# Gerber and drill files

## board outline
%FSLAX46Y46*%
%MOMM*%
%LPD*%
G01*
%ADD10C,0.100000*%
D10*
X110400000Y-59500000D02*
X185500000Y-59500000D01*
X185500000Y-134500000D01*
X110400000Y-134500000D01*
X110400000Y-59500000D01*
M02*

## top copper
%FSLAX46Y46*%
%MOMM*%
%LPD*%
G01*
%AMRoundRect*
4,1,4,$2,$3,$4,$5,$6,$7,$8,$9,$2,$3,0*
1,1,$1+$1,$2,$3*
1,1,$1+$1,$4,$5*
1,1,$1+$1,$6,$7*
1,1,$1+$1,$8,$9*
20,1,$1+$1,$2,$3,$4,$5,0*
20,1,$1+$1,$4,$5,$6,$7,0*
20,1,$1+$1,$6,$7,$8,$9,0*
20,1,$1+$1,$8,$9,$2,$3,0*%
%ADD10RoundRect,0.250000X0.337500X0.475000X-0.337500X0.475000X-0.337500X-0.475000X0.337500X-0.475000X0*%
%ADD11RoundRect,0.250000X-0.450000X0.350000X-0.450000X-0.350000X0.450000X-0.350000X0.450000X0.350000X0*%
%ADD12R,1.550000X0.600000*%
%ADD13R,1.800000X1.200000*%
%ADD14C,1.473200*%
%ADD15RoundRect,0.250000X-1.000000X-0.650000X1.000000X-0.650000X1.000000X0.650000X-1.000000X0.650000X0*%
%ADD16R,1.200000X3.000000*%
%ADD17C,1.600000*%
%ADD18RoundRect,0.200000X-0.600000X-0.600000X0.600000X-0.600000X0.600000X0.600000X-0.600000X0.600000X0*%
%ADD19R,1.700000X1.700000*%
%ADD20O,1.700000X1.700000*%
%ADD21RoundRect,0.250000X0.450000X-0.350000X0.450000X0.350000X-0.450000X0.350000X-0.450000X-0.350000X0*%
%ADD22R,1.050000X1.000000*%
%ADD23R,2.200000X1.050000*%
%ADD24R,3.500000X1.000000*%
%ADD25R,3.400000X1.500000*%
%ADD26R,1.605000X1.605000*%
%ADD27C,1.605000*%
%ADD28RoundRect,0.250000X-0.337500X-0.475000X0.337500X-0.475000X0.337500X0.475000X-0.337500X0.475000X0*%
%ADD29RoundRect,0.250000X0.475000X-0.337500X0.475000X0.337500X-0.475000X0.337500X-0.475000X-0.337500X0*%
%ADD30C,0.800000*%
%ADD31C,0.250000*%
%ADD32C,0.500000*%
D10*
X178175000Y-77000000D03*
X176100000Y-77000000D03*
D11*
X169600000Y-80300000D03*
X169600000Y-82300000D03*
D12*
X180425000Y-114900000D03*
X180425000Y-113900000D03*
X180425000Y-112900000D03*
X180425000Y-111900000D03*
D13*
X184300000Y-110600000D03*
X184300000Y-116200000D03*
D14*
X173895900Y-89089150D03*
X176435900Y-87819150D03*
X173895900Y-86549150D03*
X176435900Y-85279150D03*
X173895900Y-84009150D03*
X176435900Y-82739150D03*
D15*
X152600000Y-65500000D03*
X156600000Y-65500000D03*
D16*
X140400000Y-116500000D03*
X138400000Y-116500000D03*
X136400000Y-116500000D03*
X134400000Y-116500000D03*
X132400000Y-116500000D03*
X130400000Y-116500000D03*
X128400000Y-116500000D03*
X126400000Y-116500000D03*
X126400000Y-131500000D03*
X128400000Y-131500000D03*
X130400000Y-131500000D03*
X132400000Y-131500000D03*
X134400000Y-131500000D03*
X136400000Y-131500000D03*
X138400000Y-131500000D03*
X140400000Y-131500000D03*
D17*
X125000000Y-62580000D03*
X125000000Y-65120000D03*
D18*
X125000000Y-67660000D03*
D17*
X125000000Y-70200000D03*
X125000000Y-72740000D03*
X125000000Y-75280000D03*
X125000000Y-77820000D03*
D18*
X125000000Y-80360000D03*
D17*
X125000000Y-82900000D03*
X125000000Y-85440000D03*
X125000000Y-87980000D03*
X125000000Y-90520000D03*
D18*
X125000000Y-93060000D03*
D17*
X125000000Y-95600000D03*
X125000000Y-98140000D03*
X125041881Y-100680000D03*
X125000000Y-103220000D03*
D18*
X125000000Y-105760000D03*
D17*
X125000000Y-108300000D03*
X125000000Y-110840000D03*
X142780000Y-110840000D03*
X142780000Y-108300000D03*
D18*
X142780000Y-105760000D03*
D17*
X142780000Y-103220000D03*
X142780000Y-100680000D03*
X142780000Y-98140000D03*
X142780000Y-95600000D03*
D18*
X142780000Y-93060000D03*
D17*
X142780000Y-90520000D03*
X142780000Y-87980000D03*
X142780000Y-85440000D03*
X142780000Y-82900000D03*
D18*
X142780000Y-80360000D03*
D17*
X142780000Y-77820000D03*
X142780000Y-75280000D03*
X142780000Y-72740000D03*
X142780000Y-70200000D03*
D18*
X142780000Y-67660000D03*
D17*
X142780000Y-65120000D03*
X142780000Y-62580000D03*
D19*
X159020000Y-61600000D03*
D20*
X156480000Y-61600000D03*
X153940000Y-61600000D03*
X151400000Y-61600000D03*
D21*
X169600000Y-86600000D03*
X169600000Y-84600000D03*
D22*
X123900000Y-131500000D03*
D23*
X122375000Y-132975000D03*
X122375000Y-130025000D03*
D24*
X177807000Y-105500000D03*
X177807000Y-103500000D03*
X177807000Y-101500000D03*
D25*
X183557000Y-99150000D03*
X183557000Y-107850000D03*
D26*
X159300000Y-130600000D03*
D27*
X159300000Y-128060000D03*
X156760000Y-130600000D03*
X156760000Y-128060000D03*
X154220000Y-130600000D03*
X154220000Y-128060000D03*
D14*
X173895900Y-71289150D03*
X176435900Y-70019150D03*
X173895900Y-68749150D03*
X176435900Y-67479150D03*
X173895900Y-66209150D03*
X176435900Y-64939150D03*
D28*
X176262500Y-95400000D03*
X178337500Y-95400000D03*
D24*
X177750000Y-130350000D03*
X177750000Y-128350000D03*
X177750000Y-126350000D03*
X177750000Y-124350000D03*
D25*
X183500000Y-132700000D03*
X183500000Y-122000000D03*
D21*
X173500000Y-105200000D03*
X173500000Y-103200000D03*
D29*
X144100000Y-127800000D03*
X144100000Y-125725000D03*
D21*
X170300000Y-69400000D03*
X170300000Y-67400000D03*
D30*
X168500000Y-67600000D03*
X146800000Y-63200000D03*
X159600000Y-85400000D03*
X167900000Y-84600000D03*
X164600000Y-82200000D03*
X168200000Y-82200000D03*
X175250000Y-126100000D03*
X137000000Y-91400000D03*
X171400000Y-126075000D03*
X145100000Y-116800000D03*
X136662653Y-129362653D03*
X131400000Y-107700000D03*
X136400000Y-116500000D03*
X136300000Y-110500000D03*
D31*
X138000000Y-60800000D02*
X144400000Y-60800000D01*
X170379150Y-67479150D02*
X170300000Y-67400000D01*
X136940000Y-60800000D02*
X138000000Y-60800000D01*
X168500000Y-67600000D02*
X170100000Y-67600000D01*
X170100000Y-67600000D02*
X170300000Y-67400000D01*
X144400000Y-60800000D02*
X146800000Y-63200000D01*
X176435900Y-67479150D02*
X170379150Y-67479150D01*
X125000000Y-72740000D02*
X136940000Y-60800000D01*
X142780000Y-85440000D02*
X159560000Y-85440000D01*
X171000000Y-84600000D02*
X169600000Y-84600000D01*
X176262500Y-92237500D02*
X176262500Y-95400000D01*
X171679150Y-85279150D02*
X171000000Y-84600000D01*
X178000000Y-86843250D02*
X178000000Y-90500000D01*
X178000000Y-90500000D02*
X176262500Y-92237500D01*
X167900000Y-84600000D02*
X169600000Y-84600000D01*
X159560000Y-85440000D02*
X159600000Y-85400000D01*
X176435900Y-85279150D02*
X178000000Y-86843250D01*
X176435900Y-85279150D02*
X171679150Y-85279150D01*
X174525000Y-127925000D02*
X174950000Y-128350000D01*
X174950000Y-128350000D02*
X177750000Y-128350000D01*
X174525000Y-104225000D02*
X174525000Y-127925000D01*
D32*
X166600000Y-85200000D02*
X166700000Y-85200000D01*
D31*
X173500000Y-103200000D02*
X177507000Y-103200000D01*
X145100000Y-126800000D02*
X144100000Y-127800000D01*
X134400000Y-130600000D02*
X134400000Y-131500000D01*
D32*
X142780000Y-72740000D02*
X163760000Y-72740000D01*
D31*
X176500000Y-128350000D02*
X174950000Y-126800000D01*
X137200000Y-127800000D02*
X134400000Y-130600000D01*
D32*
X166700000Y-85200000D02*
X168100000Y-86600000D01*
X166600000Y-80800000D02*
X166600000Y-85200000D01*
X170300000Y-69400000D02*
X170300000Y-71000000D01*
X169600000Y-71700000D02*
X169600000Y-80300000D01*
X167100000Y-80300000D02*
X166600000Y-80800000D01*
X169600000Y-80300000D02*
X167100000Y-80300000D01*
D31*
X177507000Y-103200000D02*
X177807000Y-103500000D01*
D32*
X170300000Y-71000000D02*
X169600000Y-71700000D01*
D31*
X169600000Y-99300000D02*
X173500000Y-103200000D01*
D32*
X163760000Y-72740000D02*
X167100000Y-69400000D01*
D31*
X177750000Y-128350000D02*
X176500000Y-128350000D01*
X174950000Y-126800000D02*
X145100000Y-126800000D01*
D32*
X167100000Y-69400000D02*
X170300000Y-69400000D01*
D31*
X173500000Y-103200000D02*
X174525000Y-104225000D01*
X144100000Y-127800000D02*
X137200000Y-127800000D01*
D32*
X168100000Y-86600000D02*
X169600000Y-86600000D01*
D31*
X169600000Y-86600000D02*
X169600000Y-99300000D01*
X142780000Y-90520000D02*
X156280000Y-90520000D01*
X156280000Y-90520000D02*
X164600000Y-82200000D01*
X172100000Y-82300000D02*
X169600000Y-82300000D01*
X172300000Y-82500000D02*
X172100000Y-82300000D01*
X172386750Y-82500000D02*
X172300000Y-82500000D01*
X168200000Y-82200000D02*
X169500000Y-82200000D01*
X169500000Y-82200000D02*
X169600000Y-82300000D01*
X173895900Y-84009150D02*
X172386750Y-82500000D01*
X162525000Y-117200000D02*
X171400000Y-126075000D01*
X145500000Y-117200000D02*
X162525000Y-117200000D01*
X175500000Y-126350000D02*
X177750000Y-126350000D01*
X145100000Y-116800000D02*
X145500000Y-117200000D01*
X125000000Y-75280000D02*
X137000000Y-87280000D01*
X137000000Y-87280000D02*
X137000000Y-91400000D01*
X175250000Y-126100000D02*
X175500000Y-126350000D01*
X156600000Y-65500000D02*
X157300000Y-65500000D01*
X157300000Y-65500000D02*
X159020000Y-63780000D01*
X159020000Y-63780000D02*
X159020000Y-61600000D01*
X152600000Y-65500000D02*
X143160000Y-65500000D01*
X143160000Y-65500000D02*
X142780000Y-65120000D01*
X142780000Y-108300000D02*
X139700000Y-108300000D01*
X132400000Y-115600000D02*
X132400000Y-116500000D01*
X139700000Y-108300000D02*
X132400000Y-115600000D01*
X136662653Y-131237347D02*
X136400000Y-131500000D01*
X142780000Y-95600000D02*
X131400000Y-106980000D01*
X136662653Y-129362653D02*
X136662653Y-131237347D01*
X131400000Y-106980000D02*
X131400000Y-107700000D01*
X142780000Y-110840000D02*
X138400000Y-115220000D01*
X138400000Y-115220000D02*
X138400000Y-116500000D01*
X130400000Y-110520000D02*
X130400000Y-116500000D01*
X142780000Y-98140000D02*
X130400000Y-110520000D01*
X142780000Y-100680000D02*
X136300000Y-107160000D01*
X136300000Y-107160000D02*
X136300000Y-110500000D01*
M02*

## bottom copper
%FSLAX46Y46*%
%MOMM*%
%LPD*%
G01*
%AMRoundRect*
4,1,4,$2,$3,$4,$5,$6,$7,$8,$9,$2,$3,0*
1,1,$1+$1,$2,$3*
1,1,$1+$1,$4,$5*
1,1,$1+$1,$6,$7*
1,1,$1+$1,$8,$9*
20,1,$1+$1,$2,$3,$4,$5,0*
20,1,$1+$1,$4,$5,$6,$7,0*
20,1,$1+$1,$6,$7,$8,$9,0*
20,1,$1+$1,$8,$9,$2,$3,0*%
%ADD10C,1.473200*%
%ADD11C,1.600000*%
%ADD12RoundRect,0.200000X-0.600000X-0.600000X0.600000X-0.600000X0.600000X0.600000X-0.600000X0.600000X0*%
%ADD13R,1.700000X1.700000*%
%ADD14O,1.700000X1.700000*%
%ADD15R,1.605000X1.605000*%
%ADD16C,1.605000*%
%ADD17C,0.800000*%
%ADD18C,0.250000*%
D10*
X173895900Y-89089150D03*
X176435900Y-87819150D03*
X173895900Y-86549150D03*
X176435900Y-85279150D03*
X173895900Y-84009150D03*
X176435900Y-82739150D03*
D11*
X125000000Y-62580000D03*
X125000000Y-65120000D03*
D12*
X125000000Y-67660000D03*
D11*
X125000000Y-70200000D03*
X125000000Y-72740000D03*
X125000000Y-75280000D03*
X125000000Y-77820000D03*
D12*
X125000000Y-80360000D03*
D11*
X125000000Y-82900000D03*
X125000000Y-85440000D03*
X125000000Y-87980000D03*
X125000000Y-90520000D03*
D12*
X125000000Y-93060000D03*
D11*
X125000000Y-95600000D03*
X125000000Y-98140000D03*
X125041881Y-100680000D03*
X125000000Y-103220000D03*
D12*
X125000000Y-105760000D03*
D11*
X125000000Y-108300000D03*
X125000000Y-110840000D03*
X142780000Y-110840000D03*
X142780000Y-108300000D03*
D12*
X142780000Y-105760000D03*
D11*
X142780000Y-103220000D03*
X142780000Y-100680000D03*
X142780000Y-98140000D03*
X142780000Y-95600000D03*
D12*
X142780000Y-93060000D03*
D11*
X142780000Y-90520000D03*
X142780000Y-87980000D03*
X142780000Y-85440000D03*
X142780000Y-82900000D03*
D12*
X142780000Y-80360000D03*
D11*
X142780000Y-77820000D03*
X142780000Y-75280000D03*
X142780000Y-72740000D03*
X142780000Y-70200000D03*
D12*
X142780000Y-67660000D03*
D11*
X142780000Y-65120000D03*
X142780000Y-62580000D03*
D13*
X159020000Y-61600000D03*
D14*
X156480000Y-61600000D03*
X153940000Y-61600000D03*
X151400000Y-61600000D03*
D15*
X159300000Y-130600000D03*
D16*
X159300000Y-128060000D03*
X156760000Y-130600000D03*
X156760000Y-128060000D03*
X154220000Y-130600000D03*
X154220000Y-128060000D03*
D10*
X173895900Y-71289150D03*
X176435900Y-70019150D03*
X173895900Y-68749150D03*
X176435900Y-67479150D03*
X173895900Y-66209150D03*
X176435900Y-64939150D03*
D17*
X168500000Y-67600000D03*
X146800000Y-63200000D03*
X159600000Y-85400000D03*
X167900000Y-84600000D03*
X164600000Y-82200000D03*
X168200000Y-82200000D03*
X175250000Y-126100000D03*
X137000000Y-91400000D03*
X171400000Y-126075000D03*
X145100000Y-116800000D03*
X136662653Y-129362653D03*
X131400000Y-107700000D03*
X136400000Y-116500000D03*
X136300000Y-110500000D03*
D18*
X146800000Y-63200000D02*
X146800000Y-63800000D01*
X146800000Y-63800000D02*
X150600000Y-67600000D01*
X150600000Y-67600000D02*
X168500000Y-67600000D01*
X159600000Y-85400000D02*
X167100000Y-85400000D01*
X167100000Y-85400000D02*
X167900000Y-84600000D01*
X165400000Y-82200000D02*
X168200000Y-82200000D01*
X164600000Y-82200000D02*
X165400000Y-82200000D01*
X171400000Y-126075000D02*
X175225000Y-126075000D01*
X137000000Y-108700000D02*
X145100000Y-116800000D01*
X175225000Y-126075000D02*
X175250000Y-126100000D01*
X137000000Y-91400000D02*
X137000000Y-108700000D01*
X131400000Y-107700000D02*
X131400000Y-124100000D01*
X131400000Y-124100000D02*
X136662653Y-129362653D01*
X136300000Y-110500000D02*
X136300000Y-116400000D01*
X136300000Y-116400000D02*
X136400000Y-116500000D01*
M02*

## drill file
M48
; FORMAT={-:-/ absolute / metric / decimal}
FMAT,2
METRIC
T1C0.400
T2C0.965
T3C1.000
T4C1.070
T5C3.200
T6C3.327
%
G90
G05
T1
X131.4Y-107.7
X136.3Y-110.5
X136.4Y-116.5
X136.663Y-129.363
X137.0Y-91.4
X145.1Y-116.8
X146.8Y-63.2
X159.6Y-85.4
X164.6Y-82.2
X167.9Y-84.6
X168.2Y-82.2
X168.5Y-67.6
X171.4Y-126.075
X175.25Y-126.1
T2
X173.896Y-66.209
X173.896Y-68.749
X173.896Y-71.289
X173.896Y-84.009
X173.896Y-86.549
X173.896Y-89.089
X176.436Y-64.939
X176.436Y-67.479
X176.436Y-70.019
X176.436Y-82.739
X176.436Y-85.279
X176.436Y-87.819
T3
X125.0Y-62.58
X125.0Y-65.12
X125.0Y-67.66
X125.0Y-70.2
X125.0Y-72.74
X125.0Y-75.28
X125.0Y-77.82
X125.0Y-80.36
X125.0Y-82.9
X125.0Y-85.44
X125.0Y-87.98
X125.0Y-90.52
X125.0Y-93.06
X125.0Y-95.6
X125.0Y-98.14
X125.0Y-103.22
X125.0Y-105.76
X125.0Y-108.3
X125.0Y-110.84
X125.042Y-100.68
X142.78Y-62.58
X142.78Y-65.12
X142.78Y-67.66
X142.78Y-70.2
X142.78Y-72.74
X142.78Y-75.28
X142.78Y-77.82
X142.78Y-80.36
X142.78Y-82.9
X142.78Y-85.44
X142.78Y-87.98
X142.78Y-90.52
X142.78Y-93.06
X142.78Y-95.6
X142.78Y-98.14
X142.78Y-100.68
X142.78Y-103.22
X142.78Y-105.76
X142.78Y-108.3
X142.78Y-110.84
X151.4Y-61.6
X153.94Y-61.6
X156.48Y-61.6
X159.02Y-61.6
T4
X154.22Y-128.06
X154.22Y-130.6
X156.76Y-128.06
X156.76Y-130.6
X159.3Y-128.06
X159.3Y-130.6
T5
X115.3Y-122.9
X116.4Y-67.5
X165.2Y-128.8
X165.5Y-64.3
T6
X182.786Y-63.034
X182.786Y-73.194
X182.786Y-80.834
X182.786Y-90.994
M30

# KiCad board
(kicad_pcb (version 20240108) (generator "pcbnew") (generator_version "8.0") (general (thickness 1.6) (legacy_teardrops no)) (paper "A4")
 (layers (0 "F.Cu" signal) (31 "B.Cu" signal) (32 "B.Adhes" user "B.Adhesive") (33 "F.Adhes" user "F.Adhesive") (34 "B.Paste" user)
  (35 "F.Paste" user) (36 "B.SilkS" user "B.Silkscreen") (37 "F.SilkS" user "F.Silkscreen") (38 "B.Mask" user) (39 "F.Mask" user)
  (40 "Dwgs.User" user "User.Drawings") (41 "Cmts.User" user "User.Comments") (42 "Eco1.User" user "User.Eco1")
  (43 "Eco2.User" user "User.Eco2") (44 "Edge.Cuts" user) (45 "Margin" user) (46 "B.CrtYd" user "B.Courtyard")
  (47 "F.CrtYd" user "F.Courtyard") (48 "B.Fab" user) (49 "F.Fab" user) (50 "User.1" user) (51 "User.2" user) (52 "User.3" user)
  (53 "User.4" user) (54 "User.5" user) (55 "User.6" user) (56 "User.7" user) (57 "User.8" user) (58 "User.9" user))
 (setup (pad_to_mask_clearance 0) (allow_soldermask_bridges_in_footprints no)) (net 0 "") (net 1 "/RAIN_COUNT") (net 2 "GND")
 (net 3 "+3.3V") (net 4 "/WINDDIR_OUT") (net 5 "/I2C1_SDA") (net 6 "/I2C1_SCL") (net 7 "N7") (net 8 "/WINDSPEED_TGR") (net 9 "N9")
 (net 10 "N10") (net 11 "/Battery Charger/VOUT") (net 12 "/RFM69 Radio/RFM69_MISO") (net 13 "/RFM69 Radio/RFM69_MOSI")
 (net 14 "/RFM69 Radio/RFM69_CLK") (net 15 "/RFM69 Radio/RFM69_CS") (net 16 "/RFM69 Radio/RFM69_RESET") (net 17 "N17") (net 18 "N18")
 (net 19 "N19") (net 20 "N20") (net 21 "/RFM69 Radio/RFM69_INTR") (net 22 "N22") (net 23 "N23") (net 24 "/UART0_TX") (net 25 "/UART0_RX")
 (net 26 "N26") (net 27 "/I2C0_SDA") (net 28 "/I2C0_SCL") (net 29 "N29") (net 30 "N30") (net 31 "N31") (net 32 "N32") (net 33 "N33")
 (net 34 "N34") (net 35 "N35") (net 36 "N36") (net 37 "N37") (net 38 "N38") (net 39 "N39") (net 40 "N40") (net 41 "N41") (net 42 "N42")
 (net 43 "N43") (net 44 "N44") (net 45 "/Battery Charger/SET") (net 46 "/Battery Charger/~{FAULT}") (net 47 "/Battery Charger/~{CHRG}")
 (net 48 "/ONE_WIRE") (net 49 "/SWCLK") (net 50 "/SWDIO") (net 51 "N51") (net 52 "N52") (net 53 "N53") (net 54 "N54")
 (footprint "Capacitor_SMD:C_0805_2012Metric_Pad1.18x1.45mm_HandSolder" (layer "F.Cu") (at 177.1375 77 180)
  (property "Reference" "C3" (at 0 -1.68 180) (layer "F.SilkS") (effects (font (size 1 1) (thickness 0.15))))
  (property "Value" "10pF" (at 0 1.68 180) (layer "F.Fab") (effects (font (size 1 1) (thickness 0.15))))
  (pad "1" smd roundrect (at -1.0375 0 180) (size 1.175 1.45) (layers "F.Cu" "F.Paste" "F.Mask") (roundrect_rratio 0.212766)
   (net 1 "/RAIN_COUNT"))
  (pad "2" smd roundrect (at 1.0375 0 180) (size 1.175 1.45) (layers "F.Cu" "F.Paste" "F.Mask") (roundrect_rratio 0.212766) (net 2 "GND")))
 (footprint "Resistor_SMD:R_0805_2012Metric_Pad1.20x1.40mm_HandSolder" (layer "F.Cu") (at 169.6 81.3 -90)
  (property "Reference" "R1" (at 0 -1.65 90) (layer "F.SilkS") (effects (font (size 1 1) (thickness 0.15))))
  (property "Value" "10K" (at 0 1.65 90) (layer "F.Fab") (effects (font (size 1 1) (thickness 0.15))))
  (pad "1" smd roundrect (at -1 0 270) (size 1.2 1.4) (layers "F.Cu" "F.Paste" "F.Mask") (roundrect_rratio 0.208333) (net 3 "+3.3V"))
  (pad "2" smd roundrect (at 1 0 270) (size 1.2 1.4) (layers "F.Cu" "F.Paste" "F.Mask") (roundrect_rratio 0.208333) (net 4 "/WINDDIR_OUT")))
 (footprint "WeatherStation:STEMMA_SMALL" (layer "F.Cu") (at 181.2 113.4 90)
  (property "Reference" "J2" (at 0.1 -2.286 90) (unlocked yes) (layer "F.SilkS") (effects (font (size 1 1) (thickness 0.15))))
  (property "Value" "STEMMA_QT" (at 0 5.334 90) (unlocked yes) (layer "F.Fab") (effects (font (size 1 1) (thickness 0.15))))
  (pad "1" smd rect (at -1.5 -0.775 90) (size 0.6 1.55) (layers "F.Cu" "F.Paste" "F.Mask") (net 2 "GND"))
  (pad "2" smd rect (at -0.5 -0.775 90) (size 0.6 1.55) (layers "F.Cu" "F.Paste" "F.Mask") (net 3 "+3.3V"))
  (pad "3" smd rect (at 0.5 -0.775 90) (size 0.6 1.55) (layers "F.Cu" "F.Paste" "F.Mask") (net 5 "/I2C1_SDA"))
  (pad "4" smd rect (at 1.5 -0.775 90) (size 0.6 1.55) (layers "F.Cu" "F.Paste" "F.Mask") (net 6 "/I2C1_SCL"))
  (pad "5" smd rect (at 2.8 3.1 90) (size 1.2 1.8) (layers "F.Cu" "F.Paste" "F.Mask"))
  (pad "6" smd rect (at -2.8 3.1 90) (size 1.2 1.8) (layers "F.Cu" "F.Paste" "F.Mask")))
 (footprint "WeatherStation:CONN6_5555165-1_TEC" (layer "F.Cu") (at 173.8959 89.08915 90)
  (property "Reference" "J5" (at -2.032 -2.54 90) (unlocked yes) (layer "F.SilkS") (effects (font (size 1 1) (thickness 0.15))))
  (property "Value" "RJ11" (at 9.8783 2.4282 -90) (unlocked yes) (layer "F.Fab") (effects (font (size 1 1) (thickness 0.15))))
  (pad "" np_thru_hole circle (at -1.905 8.89 90) (size 3.3274 3.3274) (drill 3.3274) (layers "*.Cu" "*.Mask"))
  (pad "" np_thru_hole circle (at 8.255 8.89 90) (size 3.3274 3.3274) (drill 3.3274) (layers "*.Cu" "*.Mask"))
  (pad "1" thru_hole circle (at 0 0 90) (size 1.4732 1.4732) (drill 0.9652) (layers "*.Cu" "*.Mask") (remove_unused_layers no) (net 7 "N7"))
  (pad "2" thru_hole circle (at 1.27 2.54 90) (size 1.4732 1.4732) (drill 0.9652) (layers "*.Cu" "*.Mask") (remove_unused_layers no)
   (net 2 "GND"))
  (pad "3" thru_hole circle (at 2.54 0 90) (size 1.4732 1.4732) (drill 0.9652) (layers "*.Cu" "*.Mask") (remove_unused_layers no)
   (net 2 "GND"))
  (pad "4" thru_hole circle (at 3.81 2.54 90) (size 1.4732 1.4732) (drill 0.9652) (layers "*.Cu" "*.Mask") (remove_unused_layers no)
   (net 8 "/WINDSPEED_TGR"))
  (pad "5" thru_hole circle (at 5.08 0 90) (size 1.4732 1.4732) (drill 0.9652) (layers "*.Cu" "*.Mask") (remove_unused_layers no)
   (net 4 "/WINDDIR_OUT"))
  (pad "6" thru_hole circle (at 6.35 2.54 90) (size 1.4732 1.4732) (drill 0.9652) (layers "*.Cu" "*.Mask") (remove_unused_layers no)
   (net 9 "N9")))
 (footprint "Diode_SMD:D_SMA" (layer "F.Cu") (at 154.6 65.5)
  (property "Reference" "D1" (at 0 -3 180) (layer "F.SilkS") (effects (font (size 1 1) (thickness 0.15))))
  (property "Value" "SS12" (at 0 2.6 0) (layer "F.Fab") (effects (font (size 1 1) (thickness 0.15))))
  (pad "1" smd roundrect (at -2 0) (size 2.5 1.8) (layers "F.Cu" "F.Paste" "F.Mask") (roundrect_rratio 0.1388888889) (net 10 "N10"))
  (pad "2" smd roundrect (at 2 0) (size 2.5 1.8) (layers "F.Cu" "F.Paste" "F.Mask") (roundrect_rratio 0.1388888889)
   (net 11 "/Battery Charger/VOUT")))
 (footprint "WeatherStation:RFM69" (layer "F.Cu") (at 133.4 124 -90)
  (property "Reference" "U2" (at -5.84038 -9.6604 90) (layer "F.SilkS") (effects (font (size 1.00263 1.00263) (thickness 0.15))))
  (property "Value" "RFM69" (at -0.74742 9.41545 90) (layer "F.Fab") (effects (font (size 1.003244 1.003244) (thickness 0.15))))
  (pad "1" smd rect (at -7.5 -7 270) (size 3 1.2) (layers "F.Cu" "F.Paste" "F.Mask") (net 2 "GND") (solder_mask_margin 0.102))
  (pad "2" smd rect (at -7.5 -5 270) (size 3 1.2) (layers "F.Cu" "F.Paste" "F.Mask") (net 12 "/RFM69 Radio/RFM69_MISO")
   (solder_mask_margin 0.102))
  (pad "3" smd rect (at -7.5 -3 270) (size 3 1.2) (layers "F.Cu" "F.Paste" "F.Mask") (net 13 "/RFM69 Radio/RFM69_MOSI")
   (solder_mask_margin 0.102))
  (pad "4" smd rect (at -7.5 -1 270) (size 3 1.2) (layers "F.Cu" "F.Paste" "F.Mask") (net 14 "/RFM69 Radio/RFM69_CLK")
   (solder_mask_margin 0.102))
  (pad "5" smd rect (at -7.5 1 270) (size 3 1.2) (layers "F.Cu" "F.Paste" "F.Mask") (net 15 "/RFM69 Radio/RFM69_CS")
   (solder_mask_margin 0.102))
  (pad "6" smd rect (at -7.5 3 270) (size 3 1.2) (layers "F.Cu" "F.Paste" "F.Mask") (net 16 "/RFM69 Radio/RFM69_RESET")
   (solder_mask_margin 0.102))
  (pad "7" smd rect (at -7.5 5 270) (size 3 1.2) (layers "F.Cu" "F.Paste" "F.Mask") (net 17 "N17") (solder_mask_margin 0.102))
  (pad "8" smd rect (at -7.5 7 270) (size 3 1.2) (layers "F.Cu" "F.Paste" "F.Mask") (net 2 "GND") (solder_mask_margin 0.102))
  (pad "9" smd rect (at 7.5 7 270) (size 3 1.2) (layers "F.Cu" "F.Paste" "F.Mask") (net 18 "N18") (solder_mask_margin 0.102))
  (pad "10" smd rect (at 7.5 5 270) (size 3 1.2) (layers "F.Cu" "F.Paste" "F.Mask") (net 2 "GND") (solder_mask_margin 0.102))
  (pad "11" smd rect (at 7.5 3 270) (size 3 1.2) (layers "F.Cu" "F.Paste" "F.Mask") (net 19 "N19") (solder_mask_margin 0.102))
  (pad "12" smd rect (at 7.5 1 270) (size 3 1.2) (layers "F.Cu" "F.Paste" "F.Mask") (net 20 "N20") (solder_mask_margin 0.102))
  (pad "13" smd rect (at 7.5 -1 270) (size 3 1.2) (layers "F.Cu" "F.Paste" "F.Mask") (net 3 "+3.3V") (solder_mask_margin 0.102))
  (pad "14" smd rect (at 7.5 -3 270) (size 3 1.2) (layers "F.Cu" "F.Paste" "F.Mask") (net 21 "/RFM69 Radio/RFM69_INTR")
   (solder_mask_margin 0.102))
  (pad "15" smd rect (at 7.5 -5 270) (size 3 1.2) (layers "F.Cu" "F.Paste" "F.Mask") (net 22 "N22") (solder_mask_margin 0.102))
  (pad "16" smd rect (at 7.5 -7 270) (size 3 1.2) (layers "F.Cu" "F.Paste" "F.Mask") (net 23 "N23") (solder_mask_margin 0.102)))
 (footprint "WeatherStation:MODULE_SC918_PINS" (layer "F.Cu") (at 133.89 86.71)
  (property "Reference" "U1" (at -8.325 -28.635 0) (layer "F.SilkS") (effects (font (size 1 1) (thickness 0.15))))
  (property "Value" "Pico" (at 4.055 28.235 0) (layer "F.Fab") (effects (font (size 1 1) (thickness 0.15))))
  (pad "1" thru_hole circle (at -8.89 -24.13) (size 1.6 1.6) (drill 1) (layers "*.Cu" "*.Mask") (remove_unused_layers no)
   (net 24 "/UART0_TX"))
  (pad "2" thru_hole circle (at -8.89 -21.59) (size 1.6 1.6) (drill 1) (layers "*.Cu" "*.Mask") (remove_unused_layers no)
   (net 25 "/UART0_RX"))
  (pad "3" thru_hole roundrect (at -8.89 -19.05) (size 1.6 1.6) (drill 1) (layers "*.Cu" "*.Mask") (remove_unused_layers no)
   (roundrect_rratio 0.125) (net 2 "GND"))
  (pad "4" thru_hole circle (at -8.89 -16.51) (size 1.6 1.6) (drill 1) (layers "*.Cu" "*.Mask") (remove_unused_layers no) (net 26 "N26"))
  (pad "5" thru_hole circle (at -8.89 -13.97) (size 1.6 1.6) (drill 1) (layers "*.Cu" "*.Mask") (remove_unused_layers no)
   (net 1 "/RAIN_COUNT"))
  (pad "6" thru_hole circle (at -8.89 -11.43) (size 1.6 1.6) (drill 1) (layers "*.Cu" "*.Mask") (remove_unused_layers no)
   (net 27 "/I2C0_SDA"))
  (pad "7" thru_hole circle (at -8.89 -8.89) (size 1.6 1.6) (drill 1) (layers "*.Cu" "*.Mask") (remove_unused_layers no)
   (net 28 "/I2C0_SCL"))
  (pad "8" thru_hole roundrect (at -8.89 -6.35) (size 1.6 1.6) (drill 1) (layers "*.Cu" "*.Mask") (remove_unused_layers no)
   (roundrect_rratio 0.125) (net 2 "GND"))
  (pad "9" thru_hole circle (at -8.89 -3.81) (size 1.6 1.6) (drill 1) (layers "*.Cu" "*.Mask") (remove_unused_layers no) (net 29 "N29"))
  (pad "10" thru_hole circle (at -8.89 -1.27) (size 1.6 1.6) (drill 1) (layers "*.Cu" "*.Mask") (remove_unused_layers no) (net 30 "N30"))
  (pad "11" thru_hole circle (at -8.89 1.27) (size 1.6 1.6) (drill 1) (layers "*.Cu" "*.Mask") (remove_unused_layers no) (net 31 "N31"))
  (pad "12" thru_hole circle (at -8.89 3.81) (size 1.6 1.6) (drill 1) (layers "*.Cu" "*.Mask") (remove_unused_layers no) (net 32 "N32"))
  (pad "13" thru_hole roundrect (at -8.89 6.35) (size 1.6 1.6) (drill 1) (layers "*.Cu" "*.Mask") (remove_unused_layers no)
   (roundrect_rratio 0.125) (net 2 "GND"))
  (pad "14" thru_hole circle (at -8.89 8.89) (size 1.6 1.6) (drill 1) (layers "*.Cu" "*.Mask") (remove_unused_layers no) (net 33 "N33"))
  (pad "15" thru_hole circle (at -8.89 11.43) (size 1.6 1.6) (drill 1) (layers "*.Cu" "*.Mask") (remove_unused_layers no) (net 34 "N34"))
  (pad "16" thru_hole circle (at -8.848119 13.97) (size 1.6 1.6) (drill 1) (layers "*.Cu" "*.Mask") (remove_unused_layers no) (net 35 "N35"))
  (pad "17" thru_hole circle (at -8.89 16.51) (size 1.6 1.6) (drill 1) (layers "*.Cu" "*.Mask") (remove_unused_layers no) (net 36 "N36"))
  (pad "18" thru_hole roundrect (at -8.89 19.05) (size 1.6 1.6) (drill 1) (layers "*.Cu" "*.Mask") (remove_unused_layers no)
   (roundrect_rratio 0.125) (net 2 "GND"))
  (pad "19" thru_hole circle (at -8.89 21.59) (size 1.6 1.6) (drill 1) (layers "*.Cu" "*.Mask") (remove_unused_layers no) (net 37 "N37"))
  (pad "20" thru_hole circle (at -8.89 24.13) (size 1.6 1.6) (drill 1) (layers "*.Cu" "*.Mask") (remove_unused_layers no) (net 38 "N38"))
  (pad "21" thru_hole circle (at 8.89 24.13) (size 1.6 1.6) (drill 1) (layers "*.Cu" "*.Mask") (remove_unused_layers no)
   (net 12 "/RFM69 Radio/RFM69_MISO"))
  (pad "22" thru_hole circle (at 8.89 21.59) (size 1.6 1.6) (drill 1) (layers "*.Cu" "*.Mask") (remove_unused_layers no)
   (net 15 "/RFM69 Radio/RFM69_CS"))
  (pad "23" thru_hole roundrect (at 8.89 19.05) (size 1.6 1.6) (drill 1) (layers "*.Cu" "*.Mask") (remove_unused_layers no)
   (roundrect_rratio 0.125) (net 2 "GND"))
  (pad "24" thru_hole circle (at 8.89 16.51) (size 1.6 1.6) (drill 1) (layers "*.Cu" "*.Mask") (remove_unused_layers no)
   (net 14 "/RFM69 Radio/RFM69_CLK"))
  (pad "25" thru_hole circle (at 8.89 13.97) (size 1.6 1.6) (drill 1) (layers "*.Cu" "*.Mask") (remove_unused_layers no)
   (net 13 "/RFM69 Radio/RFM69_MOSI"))
  (pad "26" thru_hole circle (at 8.89 11.43) (size 1.6 1.6) (drill 1) (layers "*.Cu" "*.Mask") (remove_unused_layers no)
   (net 16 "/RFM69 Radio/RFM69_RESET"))
  (pad "27" thru_hole circle (at 8.89 8.89) (size 1.6 1.6) (drill 1) (layers "*.Cu" "*.Mask") (remove_unused_layers no)
   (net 21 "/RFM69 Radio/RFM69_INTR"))
  (pad "28" thru_hole roundrect (at 8.89 6.35) (size 1.6 1.6) (drill 1) (layers "*.Cu" "*.Mask") (remove_unused_layers no)
   (roundrect_rratio 0.125) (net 2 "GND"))
  (pad "29" thru_hole circle (at 8.89 3.81) (size 1.6 1.6) (drill 1) (layers "*.Cu" "*.Mask") (remove_unused_layers no)
   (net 4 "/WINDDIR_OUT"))
  (pad "30" thru_hole circle (at 8.89 1.27) (size 1.6 1.6) (drill 1) (layers "*.Cu" "*.Mask") (remove_unused_layers no) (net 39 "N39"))
  (pad "31" thru_hole circle (at 8.89 -1.27) (size 1.6 1.6) (drill 1) (layers "*.Cu" "*.Mask") (remove_unused_layers no)
   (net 8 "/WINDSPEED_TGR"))
  (pad "32" thru_hole circle (at 8.89 -3.81) (size 1.6 1.6) (drill 1) (layers "*.Cu" "*.Mask") (remove_unused_layers no) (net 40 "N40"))
  (pad "33" thru_hole roundrect (at 8.89 -6.35) (size 1.6 1.6) (drill 1) (layers "*.Cu" "*.Mask") (remove_unused_layers no)
   (roundrect_rratio 0.125) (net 2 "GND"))
  (pad "34" thru_hole circle (at 8.89 -8.89) (size 1.6 1.6) (drill 1) (layers "*.Cu" "*.Mask") (remove_unused_layers no) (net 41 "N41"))
  (pad "35" thru_hole circle (at 8.89 -11.43) (size 1.6 1.6) (drill 1) (layers "*.Cu" "*.Mask") (remove_unused_layers no) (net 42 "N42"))
  (pad "36" thru_hole circle (at 8.89 -13.97) (size 1.6 1.6) (drill 1) (layers "*.Cu" "*.Mask") (remove_unused_layers no) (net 3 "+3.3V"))
  (pad "37" thru_hole circle (at 8.89 -16.51) (size 1.6 1.6) (drill 1) (layers "*.Cu" "*.Mask") (remove_unused_layers no) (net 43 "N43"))
  (pad "38" thru_hole roundrect (at 8.89 -19.05) (size 1.6 1.6) (drill 1) (layers "*.Cu" "*.Mask") (remove_unused_layers no)
   (roundrect_rratio 0.125) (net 2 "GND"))
  (pad "39" thru_hole circle (at 8.89 -21.59) (size 1.6 1.6) (drill 1) (layers "*.Cu" "*.Mask") (remove_unused_layers no) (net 10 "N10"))
  (pad "40" thru_hole circle (at 8.89 -24.13) (size 1.6 1.6) (drill 1) (layers "*.Cu" "*.Mask") (remove_unused_layers no) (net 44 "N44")))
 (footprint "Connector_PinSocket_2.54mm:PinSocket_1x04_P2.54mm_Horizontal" (layer "F.Cu") (at 159.02 61.6 -90)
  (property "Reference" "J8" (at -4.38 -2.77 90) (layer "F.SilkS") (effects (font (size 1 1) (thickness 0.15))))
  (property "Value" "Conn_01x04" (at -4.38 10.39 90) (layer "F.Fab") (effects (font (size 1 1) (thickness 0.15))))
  (pad "1" thru_hole rect (at 0 0 270) (size 1.7 1.7) (drill 1) (layers "*.Cu" "*.Mask") (remove_unused_layers no)
   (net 11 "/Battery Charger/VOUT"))
  (pad "2" thru_hole oval (at 0 2.54 270) (size 1.7 1.7) (drill 1) (layers "*.Cu" "*.Mask") (remove_unused_layers no)
   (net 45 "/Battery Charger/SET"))
  (pad "3" thru_hole oval (at 0 5.08 270) (size 1.7 1.7) (drill 1) (layers "*.Cu" "*.Mask") (remove_unused_layers no)
   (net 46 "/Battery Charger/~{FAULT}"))
  (pad "4" thru_hole oval (at 0 7.62 270) (size 1.7 1.7) (drill 1) (layers "*.Cu" "*.Mask") (remove_unused_layers no)
   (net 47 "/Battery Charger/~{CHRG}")))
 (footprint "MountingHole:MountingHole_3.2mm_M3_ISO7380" (layer "F.Cu") (at 165.2 128.8)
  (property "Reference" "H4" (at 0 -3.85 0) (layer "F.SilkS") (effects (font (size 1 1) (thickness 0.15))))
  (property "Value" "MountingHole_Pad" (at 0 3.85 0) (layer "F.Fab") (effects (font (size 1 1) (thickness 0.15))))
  (pad "" np_thru_hole circle (at 0 0) (size 3.2 3.2) (drill 3.2) (layers "*.Cu" "*.Mask")))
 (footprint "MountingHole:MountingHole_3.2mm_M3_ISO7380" (layer "F.Cu") (at 115.3 122.9)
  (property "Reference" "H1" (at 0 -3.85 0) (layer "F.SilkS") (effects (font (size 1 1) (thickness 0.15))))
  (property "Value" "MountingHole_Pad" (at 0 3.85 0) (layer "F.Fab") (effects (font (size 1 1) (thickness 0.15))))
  (pad "" np_thru_hole circle (at 0 0) (size 3.2 3.2) (drill 3.2) (layers "*.Cu" "*.Mask")))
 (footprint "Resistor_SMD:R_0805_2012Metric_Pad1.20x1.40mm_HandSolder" (layer "F.Cu") (at 169.6 85.6 90)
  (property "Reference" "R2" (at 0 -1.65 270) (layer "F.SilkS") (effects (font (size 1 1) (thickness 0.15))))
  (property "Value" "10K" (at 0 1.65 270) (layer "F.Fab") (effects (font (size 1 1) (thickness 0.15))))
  (pad "1" smd roundrect (at -1 0 90) (size 1.2 1.4) (layers "F.Cu" "F.Paste" "F.Mask") (roundrect_rratio 0.208333) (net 3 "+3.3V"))
  (pad "2" smd roundrect (at 1 0 90) (size 1.2 1.4) (layers "F.Cu" "F.Paste" "F.Mask") (roundrect_rratio 0.208333) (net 8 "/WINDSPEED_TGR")))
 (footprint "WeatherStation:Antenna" (layer "F.Cu") (at 122.375 131.5 90)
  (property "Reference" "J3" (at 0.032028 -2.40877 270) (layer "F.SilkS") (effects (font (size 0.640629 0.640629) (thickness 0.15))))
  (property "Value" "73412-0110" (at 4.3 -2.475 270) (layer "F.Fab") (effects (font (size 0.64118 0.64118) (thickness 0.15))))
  (pad "1" smd rect (at 0 1.525 90) (size 1 1.05) (layers "F.Cu" "F.Paste" "F.Mask") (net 18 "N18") (solder_mask_margin 0.102))
  (pad "2" smd rect (at -1.475 0 90) (size 1.05 2.2) (layers "F.Cu" "F.Paste" "F.Mask") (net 2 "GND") (solder_mask_margin 0.102))
  (pad "3" smd rect (at 1.475 0 90) (size 1.05 2.2) (layers "F.Cu" "F.Paste" "F.Mask") (solder_mask_margin 0.102)))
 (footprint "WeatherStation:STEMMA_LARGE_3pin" (layer "F.Cu") (at 179.557 103.5 90)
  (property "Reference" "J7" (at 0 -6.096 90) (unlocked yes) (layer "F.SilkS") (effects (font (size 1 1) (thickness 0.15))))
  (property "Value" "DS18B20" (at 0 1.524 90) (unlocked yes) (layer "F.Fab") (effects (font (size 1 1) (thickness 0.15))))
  (pad "1" smd rect (at -2 -1.75 90) (size 1 3.5) (layers "F.Cu" "F.Paste" "F.Mask") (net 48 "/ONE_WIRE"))
  (pad "2" smd rect (at 0 -1.75 90) (size 1 3.5) (layers "F.Cu" "F.Paste" "F.Mask") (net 3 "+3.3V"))
  (pad "3" smd rect (at 2 -1.75 90) (size 1 3.5) (layers "F.Cu" "F.Paste" "F.Mask") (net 2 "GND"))
  (pad "4" smd rect (at 4.35 4 90) (size 1.5 3.4) (layers "F.Cu" "F.Paste" "F.Mask"))
  (pad "5" smd rect (at -4.35 4 90) (size 1.5 3.4) (layers "F.Cu" "F.Paste" "F.Mask")))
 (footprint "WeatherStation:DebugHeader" (layer "F.Cu") (at 156.76 129.33)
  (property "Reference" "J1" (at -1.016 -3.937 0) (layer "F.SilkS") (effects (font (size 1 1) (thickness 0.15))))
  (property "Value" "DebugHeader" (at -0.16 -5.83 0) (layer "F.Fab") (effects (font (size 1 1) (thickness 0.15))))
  (pad "1" thru_hole rect (at 2.54 1.27) (size 1.605 1.605) (drill 1.07) (layers "*.Cu" "*.Mask") (remove_unused_layers no)
   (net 24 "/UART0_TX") (solder_mask_margin 0.102))
  (pad "2" thru_hole circle (at 2.54 -1.27) (size 1.605 1.605) (drill 1.07) (layers "*.Cu" "*.Mask") (remove_unused_layers no)
   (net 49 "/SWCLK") (solder_mask_margin 0.102))
  (pad "3" thru_hole circle (at 0 1.27) (size 1.605 1.605) (drill 1.07) (layers "*.Cu" "*.Mask") (remove_unused_layers no)
   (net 25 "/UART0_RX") (solder_mask_margin 0.102))
  (pad "4" thru_hole circle (at 0 -1.27) (size 1.605 1.605) (drill 1.07) (layers "*.Cu" "*.Mask") (remove_unused_layers no)
   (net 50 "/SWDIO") (solder_mask_margin 0.102))
  (pad "5" thru_hole circle (at -2.54 1.27) (size 1.605 1.605) (drill 1.07) (layers "*.Cu" "*.Mask") (remove_unused_layers no) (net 2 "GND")
   (solder_mask_margin 0.102))
  (pad "6" thru_hole circle (at -2.54 -1.27) (size 1.605 1.605) (drill 1.07) (layers "*.Cu" "*.Mask") (remove_unused_layers no)
   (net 2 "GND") (solder_mask_margin 0.102)))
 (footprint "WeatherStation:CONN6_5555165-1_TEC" (layer "F.Cu") (at 173.8959 71.28915 90)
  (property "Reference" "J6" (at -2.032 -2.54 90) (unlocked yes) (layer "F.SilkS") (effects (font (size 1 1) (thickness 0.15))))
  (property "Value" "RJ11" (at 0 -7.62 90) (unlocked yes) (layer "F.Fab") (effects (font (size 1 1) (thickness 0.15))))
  (pad "" np_thru_hole circle (at -1.905 8.89 90) (size 3.3274 3.3274) (drill 3.3274) (layers "*.Cu" "*.Mask"))
  (pad "" np_thru_hole circle (at 8.255 8.89 90) (size 3.3274 3.3274) (drill 3.3274) (layers "*.Cu" "*.Mask"))
  (pad "1" thru_hole circle (at 0 0 90) (size 1.4732 1.4732) (drill 0.9652) (layers "*.Cu" "*.Mask") (remove_unused_layers no)
   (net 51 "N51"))
  (pad "2" thru_hole circle (at 1.27 2.54 90) (size 1.4732 1.4732) (drill 0.9652) (layers "*.Cu" "*.Mask") (remove_unused_layers no)
   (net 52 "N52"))
  (pad "3" thru_hole circle (at 2.54 0 90) (size 1.4732 1.4732) (drill 0.9652) (layers "*.Cu" "*.Mask") (remove_unused_layers no)
   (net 2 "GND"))
  (pad "4" thru_hole circle (at 3.81 2.54 90) (size 1.4732 1.4732) (drill 0.9652) (layers "*.Cu" "*.Mask") (remove_unused_layers no)
   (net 1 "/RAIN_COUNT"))
  (pad "5" thru_hole circle (at 5.08 0 90) (size 1.4732 1.4732) (drill 0.9652) (layers "*.Cu" "*.Mask") (remove_unused_layers no)
   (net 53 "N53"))
  (pad "6" thru_hole circle (at 6.35 2.54 90) (size 1.4732 1.4732) (drill 0.9652) (layers "*.Cu" "*.Mask") (remove_unused_layers no)
   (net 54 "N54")))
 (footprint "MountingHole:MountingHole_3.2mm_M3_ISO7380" (layer "F.Cu") (at 165.5 64.3)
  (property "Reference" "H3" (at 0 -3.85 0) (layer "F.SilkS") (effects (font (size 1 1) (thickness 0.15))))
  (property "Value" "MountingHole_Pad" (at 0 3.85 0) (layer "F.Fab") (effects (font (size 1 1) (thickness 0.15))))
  (pad "" np_thru_hole circle (at 0 0) (size 3.2 3.2) (drill 3.2) (layers "*.Cu" "*.Mask")))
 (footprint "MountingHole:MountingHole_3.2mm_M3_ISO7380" (layer "F.Cu") (at 116.4 67.5)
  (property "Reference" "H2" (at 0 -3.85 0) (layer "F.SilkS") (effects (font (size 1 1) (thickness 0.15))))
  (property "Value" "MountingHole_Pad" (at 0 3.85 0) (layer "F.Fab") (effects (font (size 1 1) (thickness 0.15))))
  (pad "" np_thru_hole circle (at 0 0) (size 3.2 3.2) (drill 3.2) (layers "*.Cu" "*.Mask")))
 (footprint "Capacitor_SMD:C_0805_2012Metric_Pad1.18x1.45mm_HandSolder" (layer "F.Cu") (at 177.3 95.4)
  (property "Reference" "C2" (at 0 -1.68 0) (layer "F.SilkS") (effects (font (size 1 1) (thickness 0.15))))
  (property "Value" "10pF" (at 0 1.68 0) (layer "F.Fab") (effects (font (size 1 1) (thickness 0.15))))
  (pad "1" smd roundrect (at -1.0375 0) (size 1.175 1.45) (layers "F.Cu" "F.Paste" "F.Mask") (roundrect_rratio 0.212766)
   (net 8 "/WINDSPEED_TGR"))
  (pad "2" smd roundrect (at 1.0375 0) (size 1.175 1.45) (layers "F.Cu" "F.Paste" "F.Mask") (roundrect_rratio 0.212766) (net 2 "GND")))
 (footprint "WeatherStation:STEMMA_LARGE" (layer "F.Cu") (at 179.5 127.35 90)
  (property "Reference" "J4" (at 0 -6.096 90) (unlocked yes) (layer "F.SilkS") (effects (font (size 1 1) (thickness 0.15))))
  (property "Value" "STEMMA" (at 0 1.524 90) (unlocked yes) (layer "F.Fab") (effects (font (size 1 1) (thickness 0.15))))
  (pad "1" smd rect (at -3 -1.75 90) (size 1 3.5) (layers "F.Cu" "F.Paste" "F.Mask") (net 2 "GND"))
  (pad "2" smd rect (at -1 -1.75 90) (size 1 3.5) (layers "F.Cu" "F.Paste" "F.Mask") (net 3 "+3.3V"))
  (pad "3" smd rect (at 1 -1.75 90) (size 1 3.5) (layers "F.Cu" "F.Paste" "F.Mask") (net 27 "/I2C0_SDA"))
  (pad "4" smd rect (at 3 -1.75 90) (size 1 3.5) (layers "F.Cu" "F.Paste" "F.Mask") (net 28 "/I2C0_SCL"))
  (pad "5" smd rect (at -5.35 4 90) (size 1.5 3.4) (layers "F.Cu" "F.Paste" "F.Mask"))
  (pad "6" smd rect (at 5.35 4 90) (size 1.5 3.4) (layers "F.Cu" "F.Paste" "F.Mask")))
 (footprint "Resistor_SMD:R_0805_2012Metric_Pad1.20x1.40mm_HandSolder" (layer "F.Cu") (at 173.5 104.2 90)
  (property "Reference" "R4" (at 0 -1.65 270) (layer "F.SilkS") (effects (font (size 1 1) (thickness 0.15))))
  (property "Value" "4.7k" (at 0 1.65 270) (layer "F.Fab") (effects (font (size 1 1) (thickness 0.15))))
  (pad "1" smd roundrect (at -1 0 90) (size 1.2 1.4) (layers "F.Cu" "F.Paste" "F.Mask") (roundrect_rratio 0.208333) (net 48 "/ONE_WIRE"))
  (pad "2" smd roundrect (at 1 0 90) (size 1.2 1.4) (layers "F.Cu" "F.Paste" "F.Mask") (roundrect_rratio 0.208333) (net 3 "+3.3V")))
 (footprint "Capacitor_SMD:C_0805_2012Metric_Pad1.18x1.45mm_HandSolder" (layer "F.Cu") (at 144.1 126.7625 90)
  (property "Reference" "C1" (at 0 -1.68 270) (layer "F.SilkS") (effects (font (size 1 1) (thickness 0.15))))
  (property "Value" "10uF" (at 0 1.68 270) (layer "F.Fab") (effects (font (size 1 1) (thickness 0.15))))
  (pad "1" smd roundrect (at -1.0375 0 90) (size 1.175 1.45) (layers "F.Cu" "F.Paste" "F.Mask") (roundrect_rratio 0.212766) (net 3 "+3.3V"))
  (pad "2" smd roundrect (at 1.0375 0 90) (size 1.175 1.45) (layers "F.Cu" "F.Paste" "F.Mask") (roundrect_rratio 0.212766) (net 2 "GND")))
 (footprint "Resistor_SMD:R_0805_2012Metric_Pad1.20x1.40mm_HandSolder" (layer "F.Cu") (at 170.3 68.4 90)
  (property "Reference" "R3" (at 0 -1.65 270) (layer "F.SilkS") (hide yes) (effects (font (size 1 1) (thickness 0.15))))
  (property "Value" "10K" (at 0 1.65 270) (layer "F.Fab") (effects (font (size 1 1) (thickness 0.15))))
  (pad "1" smd roundrect (at -1 0 90) (size 1.2 1.4) (layers "F.Cu" "F.Paste" "F.Mask") (roundrect_rratio 0.208333) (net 3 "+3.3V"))
  (pad "2" smd roundrect (at 1 0 90) (size 1.2 1.4) (layers "F.Cu" "F.Paste" "F.Mask") (roundrect_rratio 0.208333) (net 1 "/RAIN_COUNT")))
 (gr_rect (start 110.4 59.5) (end 185.5 134.5) (stroke (width 0.1) (type default)) (fill none) (layer "Edge.Cuts"))
 (segment (start 138 60.8) (end 144.4 60.8) (width 0.25) (layer "F.Cu") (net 1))
 (segment (start 170.37915 67.47915) (end 170.3 67.4) (width 0.25) (layer "F.Cu") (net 1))
 (segment (start 136.94 60.8) (end 138 60.8) (width 0.25) (layer "F.Cu") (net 1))
 (segment (start 168.5 67.6) (end 170.1 67.6) (width 0.25) (layer "F.Cu") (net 1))
 (segment (start 170.1 67.6) (end 170.3 67.4) (width 0.25) (layer "F.Cu") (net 1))
 (segment (start 144.4 60.8) (end 146.8 63.2) (width 0.25) (layer "F.Cu") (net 1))
 (segment (start 176.4359 67.47915) (end 170.37915 67.47915) (width 0.25) (layer "F.Cu") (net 1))
 (segment (start 125 72.74) (end 136.94 60.8) (width 0.25) (layer "F.Cu") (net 1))
 (via (at 168.5 67.6) (size 0.8) (drill 0.4) (layers "F.Cu" "B.Cu") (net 1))
 (via (at 146.8 63.2) (size 0.8) (drill 0.4) (layers "F.Cu" "B.Cu") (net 1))
 (segment (start 146.8 63.2) (end 146.8 63.8) (width 0.25) (layer "B.Cu") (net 1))
 (segment (start 146.8 63.8) (end 150.6 67.6) (width 0.25) (layer "B.Cu") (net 1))
 (segment (start 150.6 67.6) (end 168.5 67.6) (width 0.25) (layer "B.Cu") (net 1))
 (segment (start 142.78 85.44) (end 159.56 85.44) (width 0.25) (layer "F.Cu") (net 8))
 (segment (start 171 84.6) (end 169.6 84.6) (width 0.25) (layer "F.Cu") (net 8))
 (segment (start 176.2625 92.2375) (end 176.2625 95.4) (width 0.25) (layer "F.Cu") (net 8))
 (segment (start 171.67915 85.27915) (end 171 84.6) (width 0.25) (layer "F.Cu") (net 8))
 (segment (start 178 86.84325) (end 178 90.5) (width 0.25) (layer "F.Cu") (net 8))
 (segment (start 178 90.5) (end 176.2625 92.2375) (width 0.25) (layer "F.Cu") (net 8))
 (segment (start 167.9 84.6) (end 169.6 84.6) (width 0.25) (layer "F.Cu") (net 8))
 (segment (start 159.56 85.44) (end 159.6 85.4) (width 0.25) (layer "F.Cu") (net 8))
 (segment (start 176.4359 85.27915) (end 178 86.84325) (width 0.25) (layer "F.Cu") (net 8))
 (segment (start 176.4359 85.27915) (end 171.67915 85.27915) (width 0.25) (layer "F.Cu") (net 8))
 (via (at 159.6 85.4) (size 0.8) (drill 0.4) (layers "F.Cu" "B.Cu") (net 8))
 (via (at 167.9 84.6) (size 0.8) (drill 0.4) (layers "F.Cu" "B.Cu") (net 8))
 (segment (start 159.6 85.4) (end 167.1 85.4) (width 0.25) (layer "B.Cu") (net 8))
 (segment (start 167.1 85.4) (end 167.9 84.6) (width 0.25) (layer "B.Cu") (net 8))
 (segment (start 174.525 127.925) (end 174.95 128.35) (width 0.25) (layer "F.Cu") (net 3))
 (segment (start 174.95 128.35) (end 177.75 128.35) (width 0.25) (layer "F.Cu") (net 3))
 (segment (start 174.525 104.225) (end 174.525 127.925) (width 0.25) (layer "F.Cu") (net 3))
 (segment (start 166.6 85.2) (end 166.7 85.2) (width 0.5) (layer "F.Cu") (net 3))
 (segment (start 173.5 103.2) (end 177.507 103.2) (width 0.25) (layer "F.Cu") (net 3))
 (segment (start 145.1 126.8) (end 144.1 127.8) (width 0.25) (layer "F.Cu") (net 3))
 (segment (start 134.4 130.6) (end 134.4 131.5) (width 0.25) (layer "F.Cu") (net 3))
 (segment (start 142.78 72.74) (end 163.76 72.74) (width 0.5) (layer "F.Cu") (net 3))
 (segment (start 176.5 128.35) (end 174.95 126.8) (width 0.25) (layer "F.Cu") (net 3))
 (segment (start 137.2 127.8) (end 134.4 130.6) (width 0.25) (layer "F.Cu") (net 3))
 (segment (start 166.7 85.2) (end 168.1 86.6) (width 0.5) (layer "F.Cu") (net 3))
 (segment (start 166.6 80.8) (end 166.6 85.2) (width 0.5) (layer "F.Cu") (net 3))
 (segment (start 170.3 69.4) (end 170.3 71) (width 0.5) (layer "F.Cu") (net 3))
 (segment (start 169.6 71.7) (end 169.6 80.3) (width 0.5) (layer "F.Cu") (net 3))
 (segment (start 167.1 80.3) (end 166.6 80.8) (width 0.5) (layer "F.Cu") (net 3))
 (segment (start 169.6 80.3) (end 167.1 80.3) (width 0.5) (layer "F.Cu") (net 3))
 (segment (start 177.507 103.2) (end 177.807 103.5) (width 0.25) (layer "F.Cu") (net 3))
 (segment (start 170.3 71) (end 169.6 71.7) (width 0.5) (layer "F.Cu") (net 3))
 (segment (start 169.6 99.3) (end 173.5 103.2) (width 0.25) (layer "F.Cu") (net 3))
 (segment (start 163.76 72.74) (end 167.1 69.4) (width 0.5) (layer "F.Cu") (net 3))
 (segment (start 177.75 128.35) (end 176.5 128.35) (width 0.25) (layer "F.Cu") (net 3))
 (segment (start 174.95 126.8) (end 145.1 126.8) (width 0.25) (layer "F.Cu") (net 3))
 (segment (start 167.1 69.4) (end 170.3 69.4) (width 0.5) (layer "F.Cu") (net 3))
 (segment (start 173.5 103.2) (end 174.525 104.225) (width 0.25) (layer "F.Cu") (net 3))
 (segment (start 144.1 127.8) (end 137.2 127.8) (width 0.25) (layer "F.Cu") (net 3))
 (segment (start 168.1 86.6) (end 169.6 86.6) (width 0.5) (layer "F.Cu") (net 3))
 (segment (start 169.6 86.6) (end 169.6 99.3) (width 0.25) (layer "F.Cu") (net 3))
 (segment (start 142.78 90.52) (end 156.28 90.52) (width 0.25) (layer "F.Cu") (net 4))
 (segment (start 156.28 90.52) (end 164.6 82.2) (width 0.25) (layer "F.Cu") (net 4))
 (segment (start 172.1 82.3) (end 169.6 82.3) (width 0.25) (layer "F.Cu") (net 4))
 (segment (start 172.3 82.5) (end 172.1 82.3) (width 0.25) (layer "F.Cu") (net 4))
 (segment (start 172.38675 82.5) (end 172.3 82.5) (width 0.25) (layer "F.Cu") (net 4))
 (segment (start 168.2 82.2) (end 169.5 82.2) (width 0.25) (layer "F.Cu") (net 4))
 (segment (start 169.5 82.2) (end 169.6 82.3) (width 0.25) (layer "F.Cu") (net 4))
 (segment (start 173.8959 84.00915) (end 172.38675 82.5) (width 0.25) (layer "F.Cu") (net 4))
 (via (at 164.6 82.2) (size 0.8) (drill 0.4) (layers "F.Cu" "B.Cu") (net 4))
 (via (at 168.2 82.2) (size 0.8) (drill 0.4) (layers "F.Cu" "B.Cu") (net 4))
 (segment (start 165.4 82.2) (end 168.2 82.2) (width 0.25) (layer "B.Cu") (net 4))
 (segment (start 164.6 82.2) (end 165.4 82.2) (width 0.25) (layer "B.Cu") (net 4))
 (segment (start 162.525 117.2) (end 171.4 126.075) (width 0.25) (layer "F.Cu") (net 27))
 (segment (start 145.5 117.2) (end 162.525 117.2) (width 0.25) (layer "F.Cu") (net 27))
 (segment (start 175.5 126.35) (end 177.75 126.35) (width 0.25) (layer "F.Cu") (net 27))
 (segment (start 145.1 116.8) (end 145.5 117.2) (width 0.25) (layer "F.Cu") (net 27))
 (segment (start 125 75.28) (end 137 87.28) (width 0.25) (layer "F.Cu") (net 27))
 (segment (start 137 87.28) (end 137 91.4) (width 0.25) (layer "F.Cu") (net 27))
 (segment (start 175.25 126.1) (end 175.5 126.35) (width 0.25) (layer "F.Cu") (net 27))
 (via (at 175.25 126.1) (size 0.8) (drill 0.4) (layers "F.Cu" "B.Cu") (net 27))
 (via (at 137 91.4) (size 0.8) (drill 0.4) (layers "F.Cu" "B.Cu") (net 27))
 (via (at 171.4 126.075) (size 0.8) (drill 0.4) (layers "F.Cu" "B.Cu") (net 27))
 (via (at 145.1 116.8) (size 0.8) (drill 0.4) (layers "F.Cu" "B.Cu") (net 27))
 (segment (start 171.4 126.075) (end 175.225 126.075) (width 0.25) (layer "B.Cu") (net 27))
 (segment (start 137 108.7) (end 145.1 116.8) (width 0.25) (layer "B.Cu") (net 27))
 (segment (start 175.225 126.075) (end 175.25 126.1) (width 0.25) (layer "B.Cu") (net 27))
 (segment (start 137 91.4) (end 137 108.7) (width 0.25) (layer "B.Cu") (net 27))
 (segment (start 156.6 65.5) (end 157.3 65.5) (width 0.25) (layer "F.Cu") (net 11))
 (segment (start 157.3 65.5) (end 159.02 63.78) (width 0.25) (layer "F.Cu") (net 11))
 (segment (start 159.02 63.78) (end 159.02 61.6) (width 0.25) (layer "F.Cu") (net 11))
 (segment (start 152.6 65.5) (end 143.16 65.5) (width 0.25) (layer "F.Cu") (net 10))
 (segment (start 143.16 65.5) (end 142.78 65.12) (width 0.25) (layer "F.Cu") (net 10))
 (segment (start 142.78 108.3) (end 139.7 108.3) (width 0.25) (layer "F.Cu") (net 15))
 (segment (start 132.4 115.6) (end 132.4 116.5) (width 0.25) (layer "F.Cu") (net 15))
 (segment (start 139.7 108.3) (end 132.4 115.6) (width 0.25) (layer "F.Cu") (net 15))
 (segment (start 136.662653 131.237347) (end 136.4 131.5) (width 0.25) (layer "F.Cu") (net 21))
 (segment (start 142.78 95.6) (end 131.4 106.98) (width 0.25) (layer "F.Cu") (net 21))
 (segment (start 136.662653 129.362653) (end 136.662653 131.237347) (width 0.25) (layer "F.Cu") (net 21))
 (segment (start 131.4 106.98) (end 131.4 107.7) (width 0.25) (layer "F.Cu") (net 21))
 (via (at 136.662653 129.362653) (size 0.8) (drill 0.4) (layers "F.Cu" "B.Cu") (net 21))
 (via (at 131.4 107.7) (size 0.8) (drill 0.4) (layers "F.Cu" "B.Cu") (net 21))
 (segment (start 131.4 107.7) (end 131.4 124.1) (width 0.25) (layer "B.Cu") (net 21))
 (segment (start 131.4 124.1) (end 136.662653 129.362653) (width 0.25) (layer "B.Cu") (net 21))
 (segment (start 142.78 110.84) (end 138.4 115.22) (width 0.25) (layer "F.Cu") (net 12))
 (segment (start 138.4 115.22) (end 138.4 116.5) (width 0.25) (layer "F.Cu") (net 12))
 (segment (start 130.4 110.52) (end 130.4 116.5) (width 0.25) (layer "F.Cu") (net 16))
 (segment (start 142.78 98.14) (end 130.4 110.52) (width 0.25) (layer "F.Cu") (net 16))
 (segment (start 142.78 100.68) (end 136.3 107.16) (width 0.25) (layer "F.Cu") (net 13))
 (segment (start 136.3 107.16) (end 136.3 110.5) (width 0.25) (layer "F.Cu") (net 13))
 (via (at 136.4 116.5) (size 0.8) (drill 0.4) (layers "F.Cu" "B.Cu") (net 13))
 (via (at 136.3 110.5) (size 0.8) (drill 0.4) (layers "F.Cu" "B.Cu") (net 13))
 (segment (start 136.3 110.5) (end 136.3 116.4) (width 0.25) (layer "B.Cu") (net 13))
 (segment (start 136.3 116.4) (end 136.4 116.5) (width 0.25) (layer "B.Cu") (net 13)))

